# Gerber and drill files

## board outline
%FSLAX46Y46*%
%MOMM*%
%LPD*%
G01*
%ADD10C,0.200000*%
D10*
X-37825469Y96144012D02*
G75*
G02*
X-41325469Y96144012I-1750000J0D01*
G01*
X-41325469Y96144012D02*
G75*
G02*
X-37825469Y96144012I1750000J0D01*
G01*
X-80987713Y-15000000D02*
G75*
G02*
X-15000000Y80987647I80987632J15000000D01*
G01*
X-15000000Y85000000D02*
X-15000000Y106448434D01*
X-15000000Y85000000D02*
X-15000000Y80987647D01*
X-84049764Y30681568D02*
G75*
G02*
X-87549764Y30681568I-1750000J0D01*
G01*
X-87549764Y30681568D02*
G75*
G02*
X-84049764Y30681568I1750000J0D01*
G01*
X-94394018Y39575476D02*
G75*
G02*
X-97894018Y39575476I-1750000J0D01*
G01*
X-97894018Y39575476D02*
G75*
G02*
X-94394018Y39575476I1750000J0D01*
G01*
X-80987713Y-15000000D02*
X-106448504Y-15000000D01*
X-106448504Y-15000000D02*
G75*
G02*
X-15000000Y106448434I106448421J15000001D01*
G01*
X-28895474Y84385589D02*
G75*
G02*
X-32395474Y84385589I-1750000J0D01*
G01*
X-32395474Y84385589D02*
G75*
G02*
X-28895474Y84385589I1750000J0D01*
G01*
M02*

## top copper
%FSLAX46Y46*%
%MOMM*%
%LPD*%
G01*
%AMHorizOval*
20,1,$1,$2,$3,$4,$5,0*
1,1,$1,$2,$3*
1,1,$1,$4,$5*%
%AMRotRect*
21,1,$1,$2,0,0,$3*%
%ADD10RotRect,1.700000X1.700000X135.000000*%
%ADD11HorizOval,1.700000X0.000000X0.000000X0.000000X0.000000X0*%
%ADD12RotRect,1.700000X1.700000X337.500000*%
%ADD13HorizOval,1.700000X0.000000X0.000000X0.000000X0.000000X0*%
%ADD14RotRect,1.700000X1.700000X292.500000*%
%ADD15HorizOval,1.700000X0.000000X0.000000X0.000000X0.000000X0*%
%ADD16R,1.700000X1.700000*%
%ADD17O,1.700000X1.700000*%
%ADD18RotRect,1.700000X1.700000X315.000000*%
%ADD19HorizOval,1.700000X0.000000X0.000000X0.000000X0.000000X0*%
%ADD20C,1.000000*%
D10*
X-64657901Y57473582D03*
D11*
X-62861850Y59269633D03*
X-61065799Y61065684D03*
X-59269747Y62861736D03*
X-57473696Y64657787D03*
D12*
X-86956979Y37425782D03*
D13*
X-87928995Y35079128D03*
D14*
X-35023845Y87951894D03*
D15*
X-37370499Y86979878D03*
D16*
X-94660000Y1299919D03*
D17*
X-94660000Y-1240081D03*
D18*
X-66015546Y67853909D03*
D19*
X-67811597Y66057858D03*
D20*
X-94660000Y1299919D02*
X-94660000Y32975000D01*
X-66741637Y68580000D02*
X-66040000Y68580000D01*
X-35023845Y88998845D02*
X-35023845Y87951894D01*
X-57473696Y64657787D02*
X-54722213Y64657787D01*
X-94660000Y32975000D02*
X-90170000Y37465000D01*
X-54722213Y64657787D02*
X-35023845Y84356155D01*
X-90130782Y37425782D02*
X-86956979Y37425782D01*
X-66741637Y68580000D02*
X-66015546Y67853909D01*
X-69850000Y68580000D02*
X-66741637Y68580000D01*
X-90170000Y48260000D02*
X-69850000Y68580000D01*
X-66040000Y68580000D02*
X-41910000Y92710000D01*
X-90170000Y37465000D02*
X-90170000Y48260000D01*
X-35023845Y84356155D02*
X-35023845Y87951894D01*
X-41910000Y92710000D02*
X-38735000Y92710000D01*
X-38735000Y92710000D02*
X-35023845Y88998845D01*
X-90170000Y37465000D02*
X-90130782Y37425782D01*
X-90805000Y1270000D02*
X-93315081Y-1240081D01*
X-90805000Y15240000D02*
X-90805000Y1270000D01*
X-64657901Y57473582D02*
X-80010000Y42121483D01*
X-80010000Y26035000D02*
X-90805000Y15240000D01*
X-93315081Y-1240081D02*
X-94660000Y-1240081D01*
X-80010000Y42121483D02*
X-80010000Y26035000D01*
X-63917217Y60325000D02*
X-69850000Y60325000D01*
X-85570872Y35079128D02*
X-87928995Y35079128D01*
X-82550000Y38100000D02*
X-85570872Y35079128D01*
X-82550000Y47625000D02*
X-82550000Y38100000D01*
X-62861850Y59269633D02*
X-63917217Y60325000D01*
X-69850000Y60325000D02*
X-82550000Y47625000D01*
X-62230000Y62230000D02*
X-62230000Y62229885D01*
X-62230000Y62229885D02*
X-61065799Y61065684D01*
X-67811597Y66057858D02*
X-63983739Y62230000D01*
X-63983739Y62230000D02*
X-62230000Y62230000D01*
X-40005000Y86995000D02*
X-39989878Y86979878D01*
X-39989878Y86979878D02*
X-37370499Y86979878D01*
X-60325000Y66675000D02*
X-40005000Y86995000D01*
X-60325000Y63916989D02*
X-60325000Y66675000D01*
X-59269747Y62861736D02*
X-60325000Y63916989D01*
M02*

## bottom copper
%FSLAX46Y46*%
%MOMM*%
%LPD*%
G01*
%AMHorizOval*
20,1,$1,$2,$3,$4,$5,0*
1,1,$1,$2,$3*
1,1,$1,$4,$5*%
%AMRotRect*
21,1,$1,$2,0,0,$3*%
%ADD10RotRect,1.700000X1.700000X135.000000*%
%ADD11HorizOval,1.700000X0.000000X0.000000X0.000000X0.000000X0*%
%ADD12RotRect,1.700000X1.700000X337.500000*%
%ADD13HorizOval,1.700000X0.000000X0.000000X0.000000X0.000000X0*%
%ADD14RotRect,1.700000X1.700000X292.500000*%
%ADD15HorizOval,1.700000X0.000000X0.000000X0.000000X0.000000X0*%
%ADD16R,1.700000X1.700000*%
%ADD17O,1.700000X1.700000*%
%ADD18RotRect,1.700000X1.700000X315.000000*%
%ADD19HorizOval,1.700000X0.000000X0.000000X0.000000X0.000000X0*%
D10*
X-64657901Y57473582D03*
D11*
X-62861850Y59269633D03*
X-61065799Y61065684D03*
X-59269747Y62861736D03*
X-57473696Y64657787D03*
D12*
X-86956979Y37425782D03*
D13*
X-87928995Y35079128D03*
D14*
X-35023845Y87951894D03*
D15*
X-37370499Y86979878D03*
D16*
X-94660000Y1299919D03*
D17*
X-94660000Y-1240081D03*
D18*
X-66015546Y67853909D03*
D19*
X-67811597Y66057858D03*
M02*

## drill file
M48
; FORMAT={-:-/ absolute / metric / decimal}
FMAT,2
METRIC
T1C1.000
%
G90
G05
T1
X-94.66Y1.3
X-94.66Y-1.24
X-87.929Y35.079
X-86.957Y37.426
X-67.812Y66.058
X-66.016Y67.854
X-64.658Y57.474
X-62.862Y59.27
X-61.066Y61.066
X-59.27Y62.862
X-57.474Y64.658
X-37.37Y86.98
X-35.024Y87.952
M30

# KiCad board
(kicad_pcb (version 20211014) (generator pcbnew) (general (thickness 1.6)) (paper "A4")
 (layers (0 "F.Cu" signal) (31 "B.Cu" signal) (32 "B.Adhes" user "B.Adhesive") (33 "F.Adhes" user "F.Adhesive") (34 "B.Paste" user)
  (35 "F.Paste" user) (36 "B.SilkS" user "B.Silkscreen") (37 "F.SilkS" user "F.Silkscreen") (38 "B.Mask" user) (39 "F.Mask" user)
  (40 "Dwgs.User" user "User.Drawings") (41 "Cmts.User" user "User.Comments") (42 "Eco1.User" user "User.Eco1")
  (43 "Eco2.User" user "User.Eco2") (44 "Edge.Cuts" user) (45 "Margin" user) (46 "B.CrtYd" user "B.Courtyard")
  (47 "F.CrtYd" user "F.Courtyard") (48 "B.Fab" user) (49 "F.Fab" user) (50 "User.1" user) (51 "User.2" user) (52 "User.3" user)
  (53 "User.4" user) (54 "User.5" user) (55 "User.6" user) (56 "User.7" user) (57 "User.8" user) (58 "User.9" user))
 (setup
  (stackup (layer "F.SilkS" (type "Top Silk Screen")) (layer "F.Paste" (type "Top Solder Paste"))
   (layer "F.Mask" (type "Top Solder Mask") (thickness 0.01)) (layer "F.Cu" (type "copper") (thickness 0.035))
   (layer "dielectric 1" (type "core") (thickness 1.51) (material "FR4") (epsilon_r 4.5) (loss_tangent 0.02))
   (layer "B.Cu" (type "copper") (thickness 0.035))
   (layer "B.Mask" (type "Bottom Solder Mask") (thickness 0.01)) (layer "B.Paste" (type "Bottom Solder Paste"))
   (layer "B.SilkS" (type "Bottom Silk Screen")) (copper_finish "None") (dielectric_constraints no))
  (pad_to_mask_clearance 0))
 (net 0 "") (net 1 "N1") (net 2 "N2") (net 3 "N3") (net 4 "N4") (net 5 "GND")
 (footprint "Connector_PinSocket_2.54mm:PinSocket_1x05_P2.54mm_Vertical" (layer "F.Cu") (at -64.657901 -57.473582 135)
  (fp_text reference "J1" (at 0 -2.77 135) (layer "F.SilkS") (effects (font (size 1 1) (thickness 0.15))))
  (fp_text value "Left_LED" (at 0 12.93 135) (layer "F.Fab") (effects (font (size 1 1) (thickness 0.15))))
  (pad "1" thru_hole rect (at 0 0 135) (size 1.7 1.7) (drill 1) (layers *.Cu *.Mask) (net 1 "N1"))
  (pad "2" thru_hole oval (at 0 2.54 135) (size 1.7 1.7) (drill 1) (layers *.Cu *.Mask) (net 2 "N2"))
  (pad "3" thru_hole oval (at 0 5.08 135) (size 1.7 1.7) (drill 1) (layers *.Cu *.Mask) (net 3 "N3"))
  (pad "4" thru_hole oval (at 0 7.62 135) (size 1.7 1.7) (drill 1) (layers *.Cu *.Mask) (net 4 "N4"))
  (pad "5" thru_hole oval (at 0 10.16 135) (size 1.7 1.7) (drill 1) (layers *.Cu *.Mask) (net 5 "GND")))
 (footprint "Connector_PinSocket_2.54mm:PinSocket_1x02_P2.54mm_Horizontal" (layer "F.Cu") (at -86.956979 -37.425782 -22.5)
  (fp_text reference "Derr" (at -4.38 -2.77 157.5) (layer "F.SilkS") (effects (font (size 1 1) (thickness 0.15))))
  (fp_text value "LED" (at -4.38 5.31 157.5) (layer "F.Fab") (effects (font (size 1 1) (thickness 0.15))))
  (pad "1" thru_hole rect (at 0 0 337.5) (size 1.7 1.7) (drill 1) (layers *.Cu *.Mask) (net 5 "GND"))
  (pad "2" thru_hole oval (at 0 2.54 337.5) (size 1.7 1.7) (drill 1) (layers *.Cu *.Mask) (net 2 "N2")))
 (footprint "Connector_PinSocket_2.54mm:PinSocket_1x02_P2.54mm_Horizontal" (layer "F.Cu") (at -35.023845 -87.951894 -67.5)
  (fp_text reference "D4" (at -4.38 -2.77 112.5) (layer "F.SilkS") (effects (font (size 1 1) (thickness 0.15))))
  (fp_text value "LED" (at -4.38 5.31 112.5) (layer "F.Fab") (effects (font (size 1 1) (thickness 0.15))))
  (pad "1" thru_hole rect (at 0 0 292.5) (size 1.7 1.7) (drill 1) (layers *.Cu *.Mask) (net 5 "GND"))
  (pad "2" thru_hole oval (at 0 2.54 292.5) (size 1.7 1.7) (drill 1) (layers *.Cu *.Mask) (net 4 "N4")))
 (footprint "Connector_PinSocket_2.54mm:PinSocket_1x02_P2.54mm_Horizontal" (layer "F.Cu") (at -94.66 -1.299919)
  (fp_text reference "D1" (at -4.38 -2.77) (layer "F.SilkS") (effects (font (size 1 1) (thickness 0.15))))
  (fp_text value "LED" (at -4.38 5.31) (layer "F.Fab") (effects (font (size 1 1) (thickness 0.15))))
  (pad "1" thru_hole rect (at 0 0) (size 1.7 1.7) (drill 1) (layers *.Cu *.Mask) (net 5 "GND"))
  (pad "2" thru_hole oval (at 0 2.54) (size 1.7 1.7) (drill 1) (layers *.Cu *.Mask) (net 1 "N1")))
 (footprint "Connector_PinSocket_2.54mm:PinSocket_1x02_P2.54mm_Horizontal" (layer "F.Cu") (at -66.015546 -67.853909 -45)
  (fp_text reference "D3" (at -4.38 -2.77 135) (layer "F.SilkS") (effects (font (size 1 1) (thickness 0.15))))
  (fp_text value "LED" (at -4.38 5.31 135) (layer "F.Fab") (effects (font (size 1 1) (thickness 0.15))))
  (pad "1" thru_hole rect (at 0 0 315) (size 1.7 1.7) (drill 1) (layers *.Cu *.Mask) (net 5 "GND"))
  (pad "2" thru_hole oval (at 0 2.54 315) (size 1.7 1.7) (drill 1) (layers *.Cu *.Mask) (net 3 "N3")))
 (gr_circle (center -39.575469 -96.144012) (end -37.825469 -96.144012) (layer "Edge.Cuts") (width 0.2) (fill none))
 (gr_arc (start -80.987713 15) (mid -67.873563 -46.660336) (end -15 -80.987647) (layer "Edge.Cuts") (width 0.2))
 (gr_line (start -15 -85) (end -15 -106.448434) (layer "Edge.Cuts") (width 0.2))
 (gr_line (start -15 -85) (end -15 -80.987647) (layer "Edge.Cuts") (width 0.2))
 (gr_circle (center -85.799764 -30.681568) (end -84.049764 -30.681568) (layer "Edge.Cuts") (width 0.2) (fill none))
 (gr_circle (center -96.144018 -39.575476) (end -94.394018 -39.575476) (layer "Edge.Cuts") (width 0.2) (fill none))
 (gr_line (start -80.987713 15) (end -106.448504 15) (layer "Edge.Cuts") (width 0.2))
 (gr_arc (start -106.448504 15) (mid -85.87706 -64.663833) (end -15 -106.448434) (layer "Edge.Cuts") (width 0.2))
 (gr_circle (center -30.645474 -84.385589) (end -28.895474 -84.385589) (layer "Edge.Cuts") (width 0.2) (fill none))
 (segment (start -94.66 -1.299919) (end -94.66 -32.975) (width 1) (layer "F.Cu") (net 5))
 (segment (start -66.741637 -68.58) (end -66.04 -68.58) (width 1) (layer "F.Cu") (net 5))
 (segment (start -35.023845 -88.998845) (end -35.023845 -87.951894) (width 1) (layer "F.Cu") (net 5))
 (segment (start -57.473696 -64.657787) (end -54.722213 -64.657787) (width 1) (layer "F.Cu") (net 5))
 (segment (start -94.66 -32.975) (end -90.17 -37.465) (width 1) (layer "F.Cu") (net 5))
 (segment (start -54.722213 -64.657787) (end -35.023845 -84.356155) (width 1) (layer "F.Cu") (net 5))
 (segment (start -90.130782 -37.425782) (end -86.956979 -37.425782) (width 1) (layer "F.Cu") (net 5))
 (segment (start -66.741637 -68.58) (end -66.015546 -67.853909) (width 1) (layer "F.Cu") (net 5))
 (segment (start -69.85 -68.58) (end -66.741637 -68.58) (width 1) (layer "F.Cu") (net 5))
 (segment (start -90.17 -48.26) (end -69.85 -68.58) (width 1) (layer "F.Cu") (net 5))
 (segment (start -66.04 -68.58) (end -41.91 -92.71) (width 1) (layer "F.Cu") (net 5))
 (segment (start -90.17 -37.465) (end -90.17 -48.26) (width 1) (layer "F.Cu") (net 5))
 (segment (start -35.023845 -84.356155) (end -35.023845 -87.951894) (width 1) (layer "F.Cu") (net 5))
 (segment (start -41.91 -92.71) (end -38.735 -92.71) (width 1) (layer "F.Cu") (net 5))
 (segment (start -38.735 -92.71) (end -35.023845 -88.998845) (width 1) (layer "F.Cu") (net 5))
 (segment (start -90.17 -37.465) (end -90.130782 -37.425782) (width 1) (layer "F.Cu") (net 5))
 (segment (start -90.805 -1.27) (end -93.315081 1.240081) (width 1) (layer "F.Cu") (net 1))
 (segment (start -90.805 -15.24) (end -90.805 -1.27) (width 1) (layer "F.Cu") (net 1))
 (segment (start -64.657901 -57.473582) (end -80.01 -42.121483) (width 1) (layer "F.Cu") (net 1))
 (segment (start -80.01 -26.035) (end -90.805 -15.24) (width 1) (layer "F.Cu") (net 1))
 (segment (start -93.315081 1.240081) (end -94.66 1.240081) (width 1) (layer "F.Cu") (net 1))
 (segment (start -80.01 -42.121483) (end -80.01 -26.035) (width 1) (layer "F.Cu") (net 1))
 (segment (start -63.917217 -60.325) (end -69.85 -60.325) (width 1) (layer "F.Cu") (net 2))
 (segment (start -85.570872 -35.079128) (end -87.928995 -35.079128) (width 1) (layer "F.Cu") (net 2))
 (segment (start -82.55 -38.1) (end -85.570872 -35.079128) (width 1) (layer "F.Cu") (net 2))
 (segment (start -82.55 -47.625) (end -82.55 -38.1) (width 1) (layer "F.Cu") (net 2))
 (segment (start -62.86185 -59.269633) (end -63.917217 -60.325) (width 1) (layer "F.Cu") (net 2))
 (segment (start -69.85 -60.325) (end -82.55 -47.625) (width 1) (layer "F.Cu") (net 2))
 (segment (start -62.23 -62.23) (end -62.23 -62.229885) (width 1) (layer "F.Cu") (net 3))
 (segment (start -62.23 -62.229885) (end -61.065799 -61.065684) (width 1) (layer "F.Cu") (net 3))
 (segment (start -67.811597 -66.057858) (end -63.983739 -62.23) (width 1) (layer "F.Cu") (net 3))
 (segment (start -63.983739 -62.23) (end -62.23 -62.23) (width 1) (layer "F.Cu") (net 3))
 (segment (start -40.005 -86.995) (end -39.989878 -86.979878) (width 1) (layer "F.Cu") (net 4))
 (segment (start -39.989878 -86.979878) (end -37.370499 -86.979878) (width 1) (layer "F.Cu") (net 4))
 (segment (start -60.325 -66.675) (end -40.005 -86.995) (width 1) (layer "F.Cu") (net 4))
 (segment (start -60.325 -63.916989) (end -60.325 -66.675) (width 1) (layer "F.Cu") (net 4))
 (segment (start -59.269747 -62.861736) (end -60.325 -63.916989) (width 1) (layer "F.Cu") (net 4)))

